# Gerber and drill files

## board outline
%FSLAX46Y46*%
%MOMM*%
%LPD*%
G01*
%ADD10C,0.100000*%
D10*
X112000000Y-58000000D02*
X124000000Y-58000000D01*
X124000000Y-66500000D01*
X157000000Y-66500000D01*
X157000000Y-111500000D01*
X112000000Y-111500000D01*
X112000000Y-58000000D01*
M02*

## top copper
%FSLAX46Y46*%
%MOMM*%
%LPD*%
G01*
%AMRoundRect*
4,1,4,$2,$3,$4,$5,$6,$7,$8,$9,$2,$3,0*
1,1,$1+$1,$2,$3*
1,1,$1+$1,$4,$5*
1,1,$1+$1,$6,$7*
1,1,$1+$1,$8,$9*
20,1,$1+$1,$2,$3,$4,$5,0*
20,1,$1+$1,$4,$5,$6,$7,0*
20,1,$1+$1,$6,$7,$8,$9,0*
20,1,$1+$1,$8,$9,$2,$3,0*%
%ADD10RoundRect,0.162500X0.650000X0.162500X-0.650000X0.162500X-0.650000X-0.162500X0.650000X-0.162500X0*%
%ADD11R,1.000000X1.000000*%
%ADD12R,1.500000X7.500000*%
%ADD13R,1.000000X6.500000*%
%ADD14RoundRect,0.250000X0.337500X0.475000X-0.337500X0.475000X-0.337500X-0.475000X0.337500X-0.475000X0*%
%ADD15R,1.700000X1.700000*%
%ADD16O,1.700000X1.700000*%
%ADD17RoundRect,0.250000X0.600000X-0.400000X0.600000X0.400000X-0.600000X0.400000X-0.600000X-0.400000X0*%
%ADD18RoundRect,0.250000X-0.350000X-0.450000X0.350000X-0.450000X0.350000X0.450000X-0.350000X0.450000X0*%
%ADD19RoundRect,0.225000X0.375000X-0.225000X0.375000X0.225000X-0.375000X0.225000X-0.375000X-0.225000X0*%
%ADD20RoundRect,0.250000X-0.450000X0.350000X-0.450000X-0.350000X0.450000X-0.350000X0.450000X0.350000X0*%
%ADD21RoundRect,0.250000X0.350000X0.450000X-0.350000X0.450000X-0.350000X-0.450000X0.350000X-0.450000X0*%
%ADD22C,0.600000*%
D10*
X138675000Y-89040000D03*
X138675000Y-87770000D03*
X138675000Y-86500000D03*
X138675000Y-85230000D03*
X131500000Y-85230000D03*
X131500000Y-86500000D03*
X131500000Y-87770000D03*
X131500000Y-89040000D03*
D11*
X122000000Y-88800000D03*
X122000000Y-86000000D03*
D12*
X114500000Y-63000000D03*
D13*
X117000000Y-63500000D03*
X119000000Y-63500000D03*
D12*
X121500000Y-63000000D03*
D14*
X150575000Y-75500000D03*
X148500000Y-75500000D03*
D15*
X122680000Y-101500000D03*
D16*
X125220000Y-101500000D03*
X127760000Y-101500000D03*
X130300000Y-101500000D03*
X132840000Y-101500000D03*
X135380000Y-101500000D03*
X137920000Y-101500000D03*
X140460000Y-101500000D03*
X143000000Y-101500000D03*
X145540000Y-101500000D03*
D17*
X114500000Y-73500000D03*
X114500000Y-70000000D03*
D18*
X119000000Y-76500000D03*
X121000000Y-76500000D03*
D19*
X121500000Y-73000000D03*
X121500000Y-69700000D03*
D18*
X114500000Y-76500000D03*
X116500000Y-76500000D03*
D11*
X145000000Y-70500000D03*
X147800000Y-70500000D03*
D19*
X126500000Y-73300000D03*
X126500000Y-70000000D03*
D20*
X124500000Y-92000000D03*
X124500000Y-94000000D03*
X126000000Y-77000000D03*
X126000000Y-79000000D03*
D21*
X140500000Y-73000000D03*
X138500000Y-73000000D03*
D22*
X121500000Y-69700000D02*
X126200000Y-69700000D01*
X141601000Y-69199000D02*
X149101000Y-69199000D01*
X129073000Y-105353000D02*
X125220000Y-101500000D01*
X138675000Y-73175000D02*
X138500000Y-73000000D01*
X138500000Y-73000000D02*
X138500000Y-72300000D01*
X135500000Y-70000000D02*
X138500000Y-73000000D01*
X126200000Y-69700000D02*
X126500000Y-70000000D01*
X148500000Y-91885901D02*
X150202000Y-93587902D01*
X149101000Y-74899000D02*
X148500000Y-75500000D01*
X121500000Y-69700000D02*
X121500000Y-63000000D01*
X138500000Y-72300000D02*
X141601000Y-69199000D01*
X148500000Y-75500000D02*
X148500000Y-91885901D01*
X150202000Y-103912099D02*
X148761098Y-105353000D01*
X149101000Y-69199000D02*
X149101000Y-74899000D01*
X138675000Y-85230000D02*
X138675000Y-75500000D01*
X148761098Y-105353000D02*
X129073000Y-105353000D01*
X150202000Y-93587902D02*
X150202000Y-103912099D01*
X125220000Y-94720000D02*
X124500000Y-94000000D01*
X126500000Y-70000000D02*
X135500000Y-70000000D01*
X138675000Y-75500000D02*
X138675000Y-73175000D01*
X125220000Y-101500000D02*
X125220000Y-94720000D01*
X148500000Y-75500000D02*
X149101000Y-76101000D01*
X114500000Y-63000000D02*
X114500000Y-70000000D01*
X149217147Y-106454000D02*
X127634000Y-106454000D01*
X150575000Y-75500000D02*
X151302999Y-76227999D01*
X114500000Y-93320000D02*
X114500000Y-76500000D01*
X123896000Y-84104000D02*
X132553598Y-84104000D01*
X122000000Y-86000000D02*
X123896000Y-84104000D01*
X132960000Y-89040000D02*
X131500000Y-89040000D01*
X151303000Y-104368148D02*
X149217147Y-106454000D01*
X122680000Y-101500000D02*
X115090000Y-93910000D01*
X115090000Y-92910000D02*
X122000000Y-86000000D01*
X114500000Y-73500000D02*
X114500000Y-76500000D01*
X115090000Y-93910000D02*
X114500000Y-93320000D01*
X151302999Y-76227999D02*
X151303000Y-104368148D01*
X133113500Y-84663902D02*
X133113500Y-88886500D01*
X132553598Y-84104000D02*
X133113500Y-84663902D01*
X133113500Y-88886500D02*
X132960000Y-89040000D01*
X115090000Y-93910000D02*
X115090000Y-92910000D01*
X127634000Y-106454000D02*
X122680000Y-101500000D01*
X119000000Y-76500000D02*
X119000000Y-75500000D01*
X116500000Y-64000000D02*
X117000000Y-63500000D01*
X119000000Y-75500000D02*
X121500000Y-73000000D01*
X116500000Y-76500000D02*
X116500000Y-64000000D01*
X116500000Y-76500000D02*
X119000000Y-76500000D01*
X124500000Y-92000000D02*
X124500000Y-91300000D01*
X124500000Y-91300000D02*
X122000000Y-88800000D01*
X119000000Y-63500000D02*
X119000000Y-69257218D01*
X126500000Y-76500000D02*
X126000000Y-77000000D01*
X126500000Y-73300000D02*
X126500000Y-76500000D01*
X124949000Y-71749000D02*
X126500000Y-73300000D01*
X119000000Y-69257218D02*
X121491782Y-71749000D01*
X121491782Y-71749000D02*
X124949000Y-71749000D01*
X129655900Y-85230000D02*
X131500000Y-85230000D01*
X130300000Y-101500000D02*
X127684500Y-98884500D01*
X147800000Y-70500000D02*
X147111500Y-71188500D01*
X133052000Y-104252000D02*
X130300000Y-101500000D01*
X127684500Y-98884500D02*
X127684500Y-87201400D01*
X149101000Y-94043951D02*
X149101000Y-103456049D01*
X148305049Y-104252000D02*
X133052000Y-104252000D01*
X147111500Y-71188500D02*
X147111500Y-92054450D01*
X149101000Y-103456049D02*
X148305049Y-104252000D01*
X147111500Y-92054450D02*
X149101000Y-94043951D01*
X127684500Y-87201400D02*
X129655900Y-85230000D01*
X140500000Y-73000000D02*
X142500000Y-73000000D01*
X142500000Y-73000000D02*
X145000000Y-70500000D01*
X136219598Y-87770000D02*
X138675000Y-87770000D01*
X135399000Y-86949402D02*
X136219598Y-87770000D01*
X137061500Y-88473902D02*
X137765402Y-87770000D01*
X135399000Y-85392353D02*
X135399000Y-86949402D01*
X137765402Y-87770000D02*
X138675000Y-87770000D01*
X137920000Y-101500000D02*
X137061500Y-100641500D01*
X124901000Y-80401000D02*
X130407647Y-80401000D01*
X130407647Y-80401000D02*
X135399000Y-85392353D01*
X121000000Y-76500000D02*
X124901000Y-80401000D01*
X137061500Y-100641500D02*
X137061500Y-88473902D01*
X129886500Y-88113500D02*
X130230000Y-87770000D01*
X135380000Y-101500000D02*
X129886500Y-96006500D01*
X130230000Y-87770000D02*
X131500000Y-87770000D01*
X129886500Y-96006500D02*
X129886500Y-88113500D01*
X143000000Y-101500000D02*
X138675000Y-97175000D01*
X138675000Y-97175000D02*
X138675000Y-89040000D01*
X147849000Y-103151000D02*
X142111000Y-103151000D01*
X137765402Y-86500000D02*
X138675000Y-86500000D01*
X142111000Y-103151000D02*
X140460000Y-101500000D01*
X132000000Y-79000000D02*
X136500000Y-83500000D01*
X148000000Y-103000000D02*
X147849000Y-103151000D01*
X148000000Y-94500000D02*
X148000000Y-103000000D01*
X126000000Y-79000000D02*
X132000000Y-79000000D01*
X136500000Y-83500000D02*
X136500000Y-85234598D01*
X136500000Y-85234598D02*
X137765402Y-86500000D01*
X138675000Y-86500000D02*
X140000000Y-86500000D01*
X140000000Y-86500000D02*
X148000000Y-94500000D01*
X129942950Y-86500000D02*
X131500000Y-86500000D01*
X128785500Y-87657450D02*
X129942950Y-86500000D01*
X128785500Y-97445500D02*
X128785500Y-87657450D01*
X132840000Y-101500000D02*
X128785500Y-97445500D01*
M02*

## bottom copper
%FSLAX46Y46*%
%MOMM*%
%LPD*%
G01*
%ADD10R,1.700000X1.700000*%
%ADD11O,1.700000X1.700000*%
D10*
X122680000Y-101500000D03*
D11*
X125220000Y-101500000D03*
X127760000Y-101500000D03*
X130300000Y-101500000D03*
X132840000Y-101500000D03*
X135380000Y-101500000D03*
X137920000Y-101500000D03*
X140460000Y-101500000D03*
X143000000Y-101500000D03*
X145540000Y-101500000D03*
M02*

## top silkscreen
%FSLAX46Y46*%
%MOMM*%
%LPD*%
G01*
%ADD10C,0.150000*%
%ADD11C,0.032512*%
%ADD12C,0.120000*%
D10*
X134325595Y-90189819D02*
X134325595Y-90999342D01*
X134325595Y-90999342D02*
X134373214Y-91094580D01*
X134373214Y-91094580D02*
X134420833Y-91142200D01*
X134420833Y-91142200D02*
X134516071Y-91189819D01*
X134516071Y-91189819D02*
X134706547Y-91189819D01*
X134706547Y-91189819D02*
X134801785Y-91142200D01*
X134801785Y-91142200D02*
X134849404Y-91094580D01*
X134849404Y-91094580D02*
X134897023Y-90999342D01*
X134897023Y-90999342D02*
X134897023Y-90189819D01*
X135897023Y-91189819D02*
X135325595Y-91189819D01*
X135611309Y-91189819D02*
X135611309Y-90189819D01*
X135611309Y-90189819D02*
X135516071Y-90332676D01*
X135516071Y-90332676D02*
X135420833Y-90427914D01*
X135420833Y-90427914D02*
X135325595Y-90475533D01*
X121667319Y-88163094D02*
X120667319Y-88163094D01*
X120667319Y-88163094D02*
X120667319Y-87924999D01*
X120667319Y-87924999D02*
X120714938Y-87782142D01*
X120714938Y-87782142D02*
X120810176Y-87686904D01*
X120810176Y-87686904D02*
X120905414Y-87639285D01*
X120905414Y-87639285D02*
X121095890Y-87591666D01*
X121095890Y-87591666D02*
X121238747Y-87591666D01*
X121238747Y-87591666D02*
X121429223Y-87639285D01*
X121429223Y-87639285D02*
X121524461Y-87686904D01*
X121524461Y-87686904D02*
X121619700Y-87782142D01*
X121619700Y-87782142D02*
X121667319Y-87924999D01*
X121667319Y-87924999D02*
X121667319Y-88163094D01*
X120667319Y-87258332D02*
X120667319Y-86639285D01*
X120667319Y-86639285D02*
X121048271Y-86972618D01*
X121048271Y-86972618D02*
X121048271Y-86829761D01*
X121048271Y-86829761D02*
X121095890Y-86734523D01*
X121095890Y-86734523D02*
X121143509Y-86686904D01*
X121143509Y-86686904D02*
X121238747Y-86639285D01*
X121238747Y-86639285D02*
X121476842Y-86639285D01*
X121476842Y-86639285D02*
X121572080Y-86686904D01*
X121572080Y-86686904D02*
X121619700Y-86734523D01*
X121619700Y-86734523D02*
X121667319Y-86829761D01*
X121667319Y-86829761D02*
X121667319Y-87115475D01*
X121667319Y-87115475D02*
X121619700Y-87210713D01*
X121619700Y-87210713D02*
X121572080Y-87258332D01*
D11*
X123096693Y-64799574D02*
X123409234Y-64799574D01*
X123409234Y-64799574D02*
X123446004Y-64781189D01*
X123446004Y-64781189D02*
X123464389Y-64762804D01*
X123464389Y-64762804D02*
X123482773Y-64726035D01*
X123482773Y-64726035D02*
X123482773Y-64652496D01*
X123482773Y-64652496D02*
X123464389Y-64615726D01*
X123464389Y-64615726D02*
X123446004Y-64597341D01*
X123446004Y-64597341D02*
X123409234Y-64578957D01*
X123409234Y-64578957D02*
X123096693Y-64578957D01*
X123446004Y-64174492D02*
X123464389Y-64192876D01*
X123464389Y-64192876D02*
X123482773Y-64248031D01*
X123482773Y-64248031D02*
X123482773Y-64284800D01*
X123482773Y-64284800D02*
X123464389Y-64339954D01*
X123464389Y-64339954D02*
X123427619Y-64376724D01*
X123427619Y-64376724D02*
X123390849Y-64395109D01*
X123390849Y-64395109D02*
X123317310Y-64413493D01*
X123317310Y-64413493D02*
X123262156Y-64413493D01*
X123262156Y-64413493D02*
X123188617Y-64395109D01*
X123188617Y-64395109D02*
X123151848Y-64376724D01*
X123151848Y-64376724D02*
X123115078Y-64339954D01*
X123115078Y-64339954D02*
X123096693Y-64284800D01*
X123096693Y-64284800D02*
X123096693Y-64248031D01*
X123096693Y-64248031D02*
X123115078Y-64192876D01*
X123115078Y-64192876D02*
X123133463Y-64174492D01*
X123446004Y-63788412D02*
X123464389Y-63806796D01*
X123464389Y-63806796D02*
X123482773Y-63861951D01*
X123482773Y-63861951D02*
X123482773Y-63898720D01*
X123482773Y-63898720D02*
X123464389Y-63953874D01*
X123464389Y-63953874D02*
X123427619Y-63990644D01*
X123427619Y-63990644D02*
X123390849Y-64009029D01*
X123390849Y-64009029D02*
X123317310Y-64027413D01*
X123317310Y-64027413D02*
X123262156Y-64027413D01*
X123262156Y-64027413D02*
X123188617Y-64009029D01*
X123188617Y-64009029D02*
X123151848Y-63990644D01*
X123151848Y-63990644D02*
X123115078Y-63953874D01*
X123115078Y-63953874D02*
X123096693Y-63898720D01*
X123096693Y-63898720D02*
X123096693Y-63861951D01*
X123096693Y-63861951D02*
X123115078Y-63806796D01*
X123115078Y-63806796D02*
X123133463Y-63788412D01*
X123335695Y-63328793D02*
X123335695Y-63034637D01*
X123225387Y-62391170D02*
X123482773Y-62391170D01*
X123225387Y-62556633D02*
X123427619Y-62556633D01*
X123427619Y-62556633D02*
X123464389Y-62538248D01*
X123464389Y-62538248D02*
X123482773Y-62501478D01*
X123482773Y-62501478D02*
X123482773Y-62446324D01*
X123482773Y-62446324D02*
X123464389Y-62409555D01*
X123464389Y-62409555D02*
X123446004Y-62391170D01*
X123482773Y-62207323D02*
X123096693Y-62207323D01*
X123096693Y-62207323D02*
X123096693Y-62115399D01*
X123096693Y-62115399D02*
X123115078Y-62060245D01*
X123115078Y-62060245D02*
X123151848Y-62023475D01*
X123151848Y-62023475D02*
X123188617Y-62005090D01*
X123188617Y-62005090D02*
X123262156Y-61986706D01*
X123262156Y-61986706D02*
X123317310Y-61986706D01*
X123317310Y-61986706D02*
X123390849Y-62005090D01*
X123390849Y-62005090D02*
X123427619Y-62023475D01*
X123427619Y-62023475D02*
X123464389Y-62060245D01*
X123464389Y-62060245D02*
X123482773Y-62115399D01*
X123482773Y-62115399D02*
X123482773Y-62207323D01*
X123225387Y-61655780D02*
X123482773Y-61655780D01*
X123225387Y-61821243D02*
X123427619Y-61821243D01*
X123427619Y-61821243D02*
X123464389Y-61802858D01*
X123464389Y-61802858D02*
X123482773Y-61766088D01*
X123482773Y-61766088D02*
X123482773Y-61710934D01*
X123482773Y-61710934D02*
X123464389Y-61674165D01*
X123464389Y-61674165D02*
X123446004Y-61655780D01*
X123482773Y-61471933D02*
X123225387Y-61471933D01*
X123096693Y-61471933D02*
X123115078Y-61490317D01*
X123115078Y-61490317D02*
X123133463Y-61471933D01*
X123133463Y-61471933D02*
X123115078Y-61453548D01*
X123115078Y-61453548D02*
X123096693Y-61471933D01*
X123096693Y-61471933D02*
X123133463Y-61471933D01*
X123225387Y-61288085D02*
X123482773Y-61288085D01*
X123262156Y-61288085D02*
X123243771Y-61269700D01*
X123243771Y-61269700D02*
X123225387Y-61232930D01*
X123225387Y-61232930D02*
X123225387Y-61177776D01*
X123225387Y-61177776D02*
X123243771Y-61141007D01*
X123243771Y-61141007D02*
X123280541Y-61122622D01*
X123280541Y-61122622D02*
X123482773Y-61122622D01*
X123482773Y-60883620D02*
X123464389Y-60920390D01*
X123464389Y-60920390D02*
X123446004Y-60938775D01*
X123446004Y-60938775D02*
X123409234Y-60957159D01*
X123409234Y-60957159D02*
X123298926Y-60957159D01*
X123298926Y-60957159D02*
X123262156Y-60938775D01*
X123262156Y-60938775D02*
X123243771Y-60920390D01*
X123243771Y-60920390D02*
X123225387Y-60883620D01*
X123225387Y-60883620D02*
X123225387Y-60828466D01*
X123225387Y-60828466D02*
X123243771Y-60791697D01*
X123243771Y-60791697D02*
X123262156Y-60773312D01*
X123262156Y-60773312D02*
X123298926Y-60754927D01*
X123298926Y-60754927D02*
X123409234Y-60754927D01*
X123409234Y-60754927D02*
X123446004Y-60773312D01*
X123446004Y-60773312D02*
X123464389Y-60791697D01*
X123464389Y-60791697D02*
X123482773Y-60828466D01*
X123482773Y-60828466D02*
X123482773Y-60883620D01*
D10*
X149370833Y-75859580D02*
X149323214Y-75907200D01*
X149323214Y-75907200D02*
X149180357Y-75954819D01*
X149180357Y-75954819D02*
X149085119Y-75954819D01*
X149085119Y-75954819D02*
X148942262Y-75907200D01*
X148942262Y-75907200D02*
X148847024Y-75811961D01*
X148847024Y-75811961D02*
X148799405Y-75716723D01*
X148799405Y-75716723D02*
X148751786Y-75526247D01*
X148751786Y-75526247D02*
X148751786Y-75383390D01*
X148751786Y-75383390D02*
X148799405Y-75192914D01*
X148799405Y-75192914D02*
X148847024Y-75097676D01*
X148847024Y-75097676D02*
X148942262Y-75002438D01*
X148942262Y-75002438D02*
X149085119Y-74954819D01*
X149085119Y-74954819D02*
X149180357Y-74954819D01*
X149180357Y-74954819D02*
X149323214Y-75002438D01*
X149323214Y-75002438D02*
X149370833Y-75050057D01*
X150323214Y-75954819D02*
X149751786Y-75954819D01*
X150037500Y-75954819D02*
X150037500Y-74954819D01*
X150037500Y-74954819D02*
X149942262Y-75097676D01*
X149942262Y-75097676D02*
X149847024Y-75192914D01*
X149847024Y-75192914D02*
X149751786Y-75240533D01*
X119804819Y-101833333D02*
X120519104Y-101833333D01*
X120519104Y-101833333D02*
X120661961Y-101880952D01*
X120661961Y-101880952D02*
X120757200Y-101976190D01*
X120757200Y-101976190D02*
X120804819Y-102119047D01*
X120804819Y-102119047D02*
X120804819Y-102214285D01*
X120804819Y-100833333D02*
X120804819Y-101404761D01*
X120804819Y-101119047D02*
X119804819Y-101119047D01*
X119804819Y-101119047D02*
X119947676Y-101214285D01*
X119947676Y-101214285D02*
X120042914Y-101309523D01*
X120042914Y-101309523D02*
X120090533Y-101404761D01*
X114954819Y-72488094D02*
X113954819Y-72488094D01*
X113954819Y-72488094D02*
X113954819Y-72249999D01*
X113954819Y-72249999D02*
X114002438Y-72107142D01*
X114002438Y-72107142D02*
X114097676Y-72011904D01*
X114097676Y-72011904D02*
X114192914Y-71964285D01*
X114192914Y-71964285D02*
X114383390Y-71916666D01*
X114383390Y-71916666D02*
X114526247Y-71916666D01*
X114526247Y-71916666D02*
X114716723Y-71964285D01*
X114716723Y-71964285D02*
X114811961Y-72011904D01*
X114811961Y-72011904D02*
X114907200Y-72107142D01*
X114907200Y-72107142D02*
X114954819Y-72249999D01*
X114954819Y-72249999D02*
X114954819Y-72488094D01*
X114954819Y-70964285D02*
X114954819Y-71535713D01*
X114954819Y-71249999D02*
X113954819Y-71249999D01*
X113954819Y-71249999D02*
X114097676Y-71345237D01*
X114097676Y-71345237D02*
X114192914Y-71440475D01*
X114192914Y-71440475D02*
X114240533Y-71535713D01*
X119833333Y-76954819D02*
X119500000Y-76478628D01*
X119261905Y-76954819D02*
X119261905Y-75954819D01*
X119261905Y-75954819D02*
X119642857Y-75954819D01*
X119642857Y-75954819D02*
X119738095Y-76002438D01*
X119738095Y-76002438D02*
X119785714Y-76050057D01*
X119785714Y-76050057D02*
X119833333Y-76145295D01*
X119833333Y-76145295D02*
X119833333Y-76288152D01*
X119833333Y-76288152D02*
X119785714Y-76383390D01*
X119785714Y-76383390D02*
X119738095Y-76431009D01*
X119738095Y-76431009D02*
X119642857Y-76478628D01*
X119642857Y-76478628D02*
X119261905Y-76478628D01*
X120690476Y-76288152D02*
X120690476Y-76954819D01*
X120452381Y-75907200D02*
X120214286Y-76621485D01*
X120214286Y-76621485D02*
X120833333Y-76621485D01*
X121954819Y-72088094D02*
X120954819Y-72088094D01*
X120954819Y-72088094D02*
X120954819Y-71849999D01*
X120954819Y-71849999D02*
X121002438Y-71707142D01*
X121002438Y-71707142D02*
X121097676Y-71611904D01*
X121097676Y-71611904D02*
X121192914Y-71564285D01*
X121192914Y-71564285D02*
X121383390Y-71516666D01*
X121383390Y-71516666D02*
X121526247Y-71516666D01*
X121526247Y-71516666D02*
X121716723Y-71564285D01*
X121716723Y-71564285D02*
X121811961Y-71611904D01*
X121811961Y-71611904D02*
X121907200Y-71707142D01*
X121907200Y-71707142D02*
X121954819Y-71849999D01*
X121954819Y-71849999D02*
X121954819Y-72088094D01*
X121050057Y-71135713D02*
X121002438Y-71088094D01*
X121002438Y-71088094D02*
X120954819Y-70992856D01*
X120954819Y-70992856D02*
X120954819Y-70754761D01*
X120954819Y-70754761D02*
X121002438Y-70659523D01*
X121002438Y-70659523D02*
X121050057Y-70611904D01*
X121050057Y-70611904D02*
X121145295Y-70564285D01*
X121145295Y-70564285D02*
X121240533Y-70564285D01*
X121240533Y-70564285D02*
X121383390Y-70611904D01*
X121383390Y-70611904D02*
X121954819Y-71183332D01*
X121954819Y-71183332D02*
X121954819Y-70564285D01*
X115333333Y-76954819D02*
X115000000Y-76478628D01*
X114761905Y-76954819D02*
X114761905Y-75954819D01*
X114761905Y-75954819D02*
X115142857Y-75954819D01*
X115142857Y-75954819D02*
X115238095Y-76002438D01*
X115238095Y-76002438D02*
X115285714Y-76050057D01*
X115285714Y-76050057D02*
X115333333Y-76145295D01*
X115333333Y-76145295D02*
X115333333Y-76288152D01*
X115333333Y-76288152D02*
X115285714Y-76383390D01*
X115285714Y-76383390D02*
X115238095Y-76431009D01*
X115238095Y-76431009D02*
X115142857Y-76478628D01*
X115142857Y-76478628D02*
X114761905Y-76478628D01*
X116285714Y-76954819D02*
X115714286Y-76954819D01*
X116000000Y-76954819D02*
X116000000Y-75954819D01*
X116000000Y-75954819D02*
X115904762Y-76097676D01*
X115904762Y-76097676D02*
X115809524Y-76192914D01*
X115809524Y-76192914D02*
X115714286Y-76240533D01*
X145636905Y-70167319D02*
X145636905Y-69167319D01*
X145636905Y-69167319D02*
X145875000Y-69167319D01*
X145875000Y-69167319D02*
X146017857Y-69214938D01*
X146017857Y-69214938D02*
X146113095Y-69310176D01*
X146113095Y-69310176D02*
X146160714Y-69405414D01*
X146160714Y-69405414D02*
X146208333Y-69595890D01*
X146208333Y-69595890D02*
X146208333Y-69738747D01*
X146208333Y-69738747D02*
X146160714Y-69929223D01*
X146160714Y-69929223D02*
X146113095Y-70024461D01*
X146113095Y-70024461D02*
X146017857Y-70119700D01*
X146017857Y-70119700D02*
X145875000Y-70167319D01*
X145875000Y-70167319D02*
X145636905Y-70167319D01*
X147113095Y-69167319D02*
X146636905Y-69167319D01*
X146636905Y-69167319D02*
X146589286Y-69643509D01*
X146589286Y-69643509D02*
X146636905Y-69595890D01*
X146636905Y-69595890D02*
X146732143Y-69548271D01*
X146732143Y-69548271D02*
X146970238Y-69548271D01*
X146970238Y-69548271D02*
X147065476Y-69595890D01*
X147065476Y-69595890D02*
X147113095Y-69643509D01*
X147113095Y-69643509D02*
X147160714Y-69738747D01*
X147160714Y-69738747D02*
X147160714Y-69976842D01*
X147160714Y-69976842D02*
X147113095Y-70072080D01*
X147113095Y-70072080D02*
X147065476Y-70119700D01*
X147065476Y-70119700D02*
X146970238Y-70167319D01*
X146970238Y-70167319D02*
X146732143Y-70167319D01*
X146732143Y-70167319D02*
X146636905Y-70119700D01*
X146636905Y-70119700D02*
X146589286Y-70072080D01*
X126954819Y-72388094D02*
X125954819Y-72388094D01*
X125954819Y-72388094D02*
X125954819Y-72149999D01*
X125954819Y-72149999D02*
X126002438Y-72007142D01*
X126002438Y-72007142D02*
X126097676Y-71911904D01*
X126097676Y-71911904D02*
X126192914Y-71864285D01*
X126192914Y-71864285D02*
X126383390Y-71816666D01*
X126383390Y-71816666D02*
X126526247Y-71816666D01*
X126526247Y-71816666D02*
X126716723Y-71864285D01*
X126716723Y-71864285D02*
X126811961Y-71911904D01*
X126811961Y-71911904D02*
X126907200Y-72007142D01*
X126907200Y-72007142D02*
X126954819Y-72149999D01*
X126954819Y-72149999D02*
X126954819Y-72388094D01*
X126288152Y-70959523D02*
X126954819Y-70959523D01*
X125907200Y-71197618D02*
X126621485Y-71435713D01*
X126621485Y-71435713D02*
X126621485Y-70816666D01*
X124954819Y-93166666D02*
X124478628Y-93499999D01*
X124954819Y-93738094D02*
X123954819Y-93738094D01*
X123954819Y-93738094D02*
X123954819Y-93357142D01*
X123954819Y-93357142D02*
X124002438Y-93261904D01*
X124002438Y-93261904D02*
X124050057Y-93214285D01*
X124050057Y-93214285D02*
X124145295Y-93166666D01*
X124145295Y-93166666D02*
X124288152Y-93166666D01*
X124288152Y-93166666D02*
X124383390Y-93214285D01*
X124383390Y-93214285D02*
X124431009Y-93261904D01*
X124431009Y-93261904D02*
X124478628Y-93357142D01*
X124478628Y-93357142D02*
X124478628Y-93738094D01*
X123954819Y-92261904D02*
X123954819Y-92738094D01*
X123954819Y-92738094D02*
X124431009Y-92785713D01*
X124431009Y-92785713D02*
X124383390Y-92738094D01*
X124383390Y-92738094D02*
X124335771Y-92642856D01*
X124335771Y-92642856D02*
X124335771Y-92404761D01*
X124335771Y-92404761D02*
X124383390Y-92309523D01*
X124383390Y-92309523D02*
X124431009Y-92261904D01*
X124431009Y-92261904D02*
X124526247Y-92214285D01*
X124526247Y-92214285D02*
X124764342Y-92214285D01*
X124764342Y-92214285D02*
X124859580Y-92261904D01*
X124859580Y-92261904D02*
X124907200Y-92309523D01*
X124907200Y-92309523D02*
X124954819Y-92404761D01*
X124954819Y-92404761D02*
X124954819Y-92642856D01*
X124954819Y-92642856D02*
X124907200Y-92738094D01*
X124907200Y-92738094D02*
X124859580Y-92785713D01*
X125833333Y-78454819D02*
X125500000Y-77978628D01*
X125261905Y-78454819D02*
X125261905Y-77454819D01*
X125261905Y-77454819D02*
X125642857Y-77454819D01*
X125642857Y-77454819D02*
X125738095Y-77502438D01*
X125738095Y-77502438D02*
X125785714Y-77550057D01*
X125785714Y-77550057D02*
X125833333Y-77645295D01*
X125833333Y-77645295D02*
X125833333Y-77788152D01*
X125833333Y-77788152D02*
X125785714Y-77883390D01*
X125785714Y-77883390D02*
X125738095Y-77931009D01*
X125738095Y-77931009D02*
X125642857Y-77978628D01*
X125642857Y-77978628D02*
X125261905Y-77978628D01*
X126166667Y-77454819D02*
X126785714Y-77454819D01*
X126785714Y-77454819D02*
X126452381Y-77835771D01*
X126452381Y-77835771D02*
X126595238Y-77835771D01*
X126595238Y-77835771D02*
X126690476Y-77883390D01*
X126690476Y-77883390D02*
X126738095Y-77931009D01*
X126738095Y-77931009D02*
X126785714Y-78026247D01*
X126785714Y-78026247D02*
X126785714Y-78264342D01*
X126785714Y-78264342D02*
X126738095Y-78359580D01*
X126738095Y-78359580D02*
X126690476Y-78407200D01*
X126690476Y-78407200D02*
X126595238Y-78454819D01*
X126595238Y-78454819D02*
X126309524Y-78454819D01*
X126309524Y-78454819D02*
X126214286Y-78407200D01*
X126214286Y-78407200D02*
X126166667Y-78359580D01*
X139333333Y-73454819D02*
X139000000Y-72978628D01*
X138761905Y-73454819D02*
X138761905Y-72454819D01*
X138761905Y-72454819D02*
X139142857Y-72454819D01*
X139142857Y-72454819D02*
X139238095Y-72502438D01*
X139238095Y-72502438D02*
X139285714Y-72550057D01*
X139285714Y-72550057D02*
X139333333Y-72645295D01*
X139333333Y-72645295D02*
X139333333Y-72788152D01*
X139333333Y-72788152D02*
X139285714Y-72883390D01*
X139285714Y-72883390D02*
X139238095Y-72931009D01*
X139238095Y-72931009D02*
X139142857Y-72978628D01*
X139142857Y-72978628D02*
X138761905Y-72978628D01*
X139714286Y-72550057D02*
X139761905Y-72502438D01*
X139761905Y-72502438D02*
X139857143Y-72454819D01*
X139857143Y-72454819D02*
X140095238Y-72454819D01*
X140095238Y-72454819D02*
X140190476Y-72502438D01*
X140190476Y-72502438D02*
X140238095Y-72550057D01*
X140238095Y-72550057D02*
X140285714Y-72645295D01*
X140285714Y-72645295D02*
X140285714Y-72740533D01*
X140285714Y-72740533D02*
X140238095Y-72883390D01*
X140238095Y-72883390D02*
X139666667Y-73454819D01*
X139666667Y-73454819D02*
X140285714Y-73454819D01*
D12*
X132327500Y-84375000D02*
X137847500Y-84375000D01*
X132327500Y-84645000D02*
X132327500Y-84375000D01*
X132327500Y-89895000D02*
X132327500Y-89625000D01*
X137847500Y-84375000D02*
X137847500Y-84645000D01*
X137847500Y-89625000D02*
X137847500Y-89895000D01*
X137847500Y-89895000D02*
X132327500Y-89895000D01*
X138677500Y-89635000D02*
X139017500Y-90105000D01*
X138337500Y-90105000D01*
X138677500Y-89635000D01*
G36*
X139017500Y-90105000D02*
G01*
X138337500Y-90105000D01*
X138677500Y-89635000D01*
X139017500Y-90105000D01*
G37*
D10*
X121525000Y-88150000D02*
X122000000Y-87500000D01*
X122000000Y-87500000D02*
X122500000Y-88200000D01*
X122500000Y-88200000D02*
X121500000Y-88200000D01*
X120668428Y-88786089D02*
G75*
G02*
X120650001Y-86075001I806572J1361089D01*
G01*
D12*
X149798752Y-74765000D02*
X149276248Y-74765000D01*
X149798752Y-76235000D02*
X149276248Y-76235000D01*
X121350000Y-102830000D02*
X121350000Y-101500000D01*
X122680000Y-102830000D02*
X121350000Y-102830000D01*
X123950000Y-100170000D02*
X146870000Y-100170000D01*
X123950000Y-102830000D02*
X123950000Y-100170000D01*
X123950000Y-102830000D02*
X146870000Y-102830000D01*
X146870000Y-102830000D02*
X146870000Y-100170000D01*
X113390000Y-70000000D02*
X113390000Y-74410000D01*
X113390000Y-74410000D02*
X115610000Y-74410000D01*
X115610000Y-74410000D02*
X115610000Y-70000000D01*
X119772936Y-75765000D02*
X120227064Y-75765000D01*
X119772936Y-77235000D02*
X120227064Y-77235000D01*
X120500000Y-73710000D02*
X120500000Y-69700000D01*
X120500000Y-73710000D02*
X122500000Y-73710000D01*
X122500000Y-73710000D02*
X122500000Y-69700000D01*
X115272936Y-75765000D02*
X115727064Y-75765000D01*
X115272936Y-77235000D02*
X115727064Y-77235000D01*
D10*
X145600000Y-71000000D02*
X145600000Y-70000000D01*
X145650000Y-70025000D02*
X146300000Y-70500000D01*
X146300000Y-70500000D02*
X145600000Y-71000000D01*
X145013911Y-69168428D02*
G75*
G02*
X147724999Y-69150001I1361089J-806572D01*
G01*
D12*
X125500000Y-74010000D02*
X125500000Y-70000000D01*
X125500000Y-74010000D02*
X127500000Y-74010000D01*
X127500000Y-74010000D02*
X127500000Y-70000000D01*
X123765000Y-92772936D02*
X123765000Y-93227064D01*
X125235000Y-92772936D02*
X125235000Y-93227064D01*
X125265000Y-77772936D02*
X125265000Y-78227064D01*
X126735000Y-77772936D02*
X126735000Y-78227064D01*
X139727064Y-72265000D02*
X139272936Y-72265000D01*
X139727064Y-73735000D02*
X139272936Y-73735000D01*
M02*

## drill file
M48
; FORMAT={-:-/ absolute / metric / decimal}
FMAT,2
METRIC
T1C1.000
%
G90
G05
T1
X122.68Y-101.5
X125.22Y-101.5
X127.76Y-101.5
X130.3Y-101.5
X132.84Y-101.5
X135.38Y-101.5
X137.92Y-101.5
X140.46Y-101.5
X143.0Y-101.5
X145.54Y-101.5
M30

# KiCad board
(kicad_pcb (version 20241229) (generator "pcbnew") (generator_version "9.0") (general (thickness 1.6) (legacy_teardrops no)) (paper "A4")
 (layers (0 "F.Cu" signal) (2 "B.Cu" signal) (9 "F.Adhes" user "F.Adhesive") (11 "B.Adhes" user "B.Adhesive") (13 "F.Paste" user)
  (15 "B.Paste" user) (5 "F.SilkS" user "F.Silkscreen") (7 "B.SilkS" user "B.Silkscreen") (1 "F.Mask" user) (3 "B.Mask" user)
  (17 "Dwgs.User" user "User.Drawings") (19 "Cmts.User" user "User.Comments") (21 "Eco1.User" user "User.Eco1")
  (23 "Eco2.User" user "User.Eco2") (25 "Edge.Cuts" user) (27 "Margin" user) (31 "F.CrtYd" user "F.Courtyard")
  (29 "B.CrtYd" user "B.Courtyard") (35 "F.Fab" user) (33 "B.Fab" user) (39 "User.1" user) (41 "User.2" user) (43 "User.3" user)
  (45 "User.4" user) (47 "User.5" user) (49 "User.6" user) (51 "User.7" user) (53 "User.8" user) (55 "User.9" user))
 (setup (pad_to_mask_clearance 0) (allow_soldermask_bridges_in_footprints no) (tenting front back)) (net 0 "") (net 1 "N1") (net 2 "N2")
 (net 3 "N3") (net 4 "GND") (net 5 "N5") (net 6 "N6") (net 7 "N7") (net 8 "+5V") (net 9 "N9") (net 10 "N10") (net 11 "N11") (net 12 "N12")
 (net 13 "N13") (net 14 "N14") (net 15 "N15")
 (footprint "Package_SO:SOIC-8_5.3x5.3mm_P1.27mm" (layer "F.Cu") (at 135.0875 87.135 180)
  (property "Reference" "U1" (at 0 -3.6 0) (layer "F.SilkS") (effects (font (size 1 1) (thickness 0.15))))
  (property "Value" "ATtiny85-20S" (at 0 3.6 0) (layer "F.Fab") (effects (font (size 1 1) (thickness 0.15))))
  (fp_line (start 2.76 2.76) (end -2.76 2.76) (stroke (width 0.12) (type solid)) (layer "F.SilkS"))
  (fp_line (start 2.76 2.49) (end 2.76 2.76) (stroke (width 0.12) (type solid)) (layer "F.SilkS"))
  (fp_line (start 2.76 -2.76) (end 2.76 -2.49) (stroke (width 0.12) (type solid)) (layer "F.SilkS"))
  (fp_line (start -2.76 2.76) (end -2.76 2.49) (stroke (width 0.12) (type solid)) (layer "F.SilkS"))
  (fp_line (start -2.76 -2.49) (end -2.76 -2.76) (stroke (width 0.12) (type solid)) (layer "F.SilkS"))
  (fp_line (start -2.76 -2.76) (end 2.76 -2.76) (stroke (width 0.12) (type solid)) (layer "F.SilkS"))
  (fp_poly (pts (xy -3.59 -2.5) (xy -3.93 -2.97) (xy -3.25 -2.97)) (stroke (width 0.12) (type solid)) (fill yes) (layer "F.SilkS"))
  (pad "1" smd roundrect (at -3.5875 -1.905 180) (size 1.625 0.65) (layers "F.Cu" "F.Mask" "F.Paste") (roundrect_rratio 0.25) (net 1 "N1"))
  (pad "2" smd roundrect (at -3.5875 -0.635 180) (size 1.625 0.65) (layers "F.Cu" "F.Mask" "F.Paste") (roundrect_rratio 0.25) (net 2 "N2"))
  (pad "3" smd roundrect (at -3.5875 0.635 180) (size 1.625 0.65) (layers "F.Cu" "F.Mask" "F.Paste") (roundrect_rratio 0.25) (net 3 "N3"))
  (pad "4" smd roundrect (at -3.5875 1.905 180) (size 1.625 0.65) (layers "F.Cu" "F.Mask" "F.Paste") (roundrect_rratio 0.25) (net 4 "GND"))
  (pad "5" smd roundrect (at 3.5875 1.905 180) (size 1.625 0.65) (layers "F.Cu" "F.Mask" "F.Paste") (roundrect_rratio 0.25) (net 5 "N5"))
  (pad "6" smd roundrect (at 3.5875 0.635 180) (size 1.625 0.65) (layers "F.Cu" "F.Mask" "F.Paste") (roundrect_rratio 0.25) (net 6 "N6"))
  (pad "7" smd roundrect (at 3.5875 -0.635 180) (size 1.625 0.65) (layers "F.Cu" "F.Mask" "F.Paste") (roundrect_rratio 0.25) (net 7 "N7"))
  (pad "8" smd roundrect (at 3.5875 -1.905 180) (size 1.625 0.65) (layers "F.Cu" "F.Mask" "F.Paste") (roundrect_rratio 0.25) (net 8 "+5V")))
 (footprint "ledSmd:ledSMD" (layer "F.Cu") (at 122 87 90)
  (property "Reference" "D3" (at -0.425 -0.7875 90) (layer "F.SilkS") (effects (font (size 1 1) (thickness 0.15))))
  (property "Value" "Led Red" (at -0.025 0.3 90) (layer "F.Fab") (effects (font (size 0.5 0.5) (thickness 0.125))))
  (fp_line (start -1.15 -0.475) (end -0.5 0) (stroke (width 0.15) (type solid)) (layer "F.SilkS"))
  (fp_line (start -0.5 0) (end -1.2 0.5) (stroke (width 0.15) (type solid)) (layer "F.SilkS"))
  (fp_line (start -1.2 0.5) (end -1.2 -0.5) (stroke (width 0.15) (type solid)) (layer "F.SilkS"))
  (fp_arc (start -1.786089 -1.331572) (mid -0.435753 -2.107089) (end 0.924999 -1.349999) (stroke (width 0.15) (type solid))
   (layer "F.SilkS"))
  (pad "1" smd rect (at -1.8 0 90) (size 1 1) (layers "F.Cu" "F.Mask" "F.Paste") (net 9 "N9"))
  (pad "2" smd rect (at 1 0 90) (size 1 1) (layers "F.Cu" "F.Mask" "F.Paste") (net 8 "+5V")))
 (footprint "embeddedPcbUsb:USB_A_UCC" (layer "F.Cu") (at 118 63.2 -90)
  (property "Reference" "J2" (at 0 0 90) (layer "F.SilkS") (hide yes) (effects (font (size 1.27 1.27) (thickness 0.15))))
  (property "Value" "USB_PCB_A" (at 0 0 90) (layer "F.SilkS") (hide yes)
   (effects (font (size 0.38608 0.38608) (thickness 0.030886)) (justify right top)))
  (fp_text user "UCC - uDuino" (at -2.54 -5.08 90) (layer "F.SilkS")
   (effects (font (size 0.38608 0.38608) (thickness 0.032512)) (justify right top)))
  (pad "1" smd rect (at -0.2 3.5 270) (size 7.5 1.5) (layers "F.Cu" "F.Mask" "F.Paste") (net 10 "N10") (solder_mask_margin 0.1016))
  (pad "2" smd rect (at 0.3 1 270) (size 6.5 1) (layers "F.Cu" "F.Mask" "F.Paste") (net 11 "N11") (solder_mask_margin 0.1016))
  (pad "3" smd rect (at 0.3 -1 270) (size 6.5 1) (layers "F.Cu" "F.Mask" "F.Paste") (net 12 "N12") (solder_mask_margin 0.1016))
  (pad "4" smd rect (at -0.2 -3.5 270) (size 7.5 1.5) (layers "F.Cu" "F.Mask" "F.Paste") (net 4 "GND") (solder_mask_margin 0.1016)))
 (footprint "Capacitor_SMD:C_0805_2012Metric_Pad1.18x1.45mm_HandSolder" (layer "F.Cu") (at 149.5375 75.5 180)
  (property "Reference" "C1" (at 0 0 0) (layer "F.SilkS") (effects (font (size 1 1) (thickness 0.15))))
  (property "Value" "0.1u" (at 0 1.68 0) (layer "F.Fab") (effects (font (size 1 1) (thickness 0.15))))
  (fp_line (start -0.261252 0.735) (end 0.261252 0.735) (stroke (width 0.12) (type solid)) (layer "F.SilkS"))
  (fp_line (start -0.261252 -0.735) (end 0.261252 -0.735) (stroke (width 0.12) (type solid)) (layer "F.SilkS"))
  (pad "1" smd roundrect (at -1.0375 0 180) (size 1.175 1.45) (layers "F.Cu" "F.Mask" "F.Paste") (roundrect_rratio 0.212766) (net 8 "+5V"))
  (pad "2" smd roundrect (at 1.0375 0 180) (size 1.175 1.45) (layers "F.Cu" "F.Mask" "F.Paste") (roundrect_rratio 0.212766) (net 4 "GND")))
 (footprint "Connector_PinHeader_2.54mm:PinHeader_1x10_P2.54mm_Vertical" (layer "F.Cu") (at 122.68 101.5 90)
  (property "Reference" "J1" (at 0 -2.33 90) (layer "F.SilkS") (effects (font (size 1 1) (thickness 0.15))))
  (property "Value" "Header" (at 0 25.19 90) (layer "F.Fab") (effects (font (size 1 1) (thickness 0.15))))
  (fp_line (start -1.33 -1.33) (end 0 -1.33) (stroke (width 0.12) (type solid)) (layer "F.SilkS"))
  (fp_line (start -1.33 0) (end -1.33 -1.33) (stroke (width 0.12) (type solid)) (layer "F.SilkS"))
  (fp_line (start 1.33 1.27) (end 1.33 24.19) (stroke (width 0.12) (type solid)) (layer "F.SilkS"))
  (fp_line (start -1.33 1.27) (end 1.33 1.27) (stroke (width 0.12) (type solid)) (layer "F.SilkS"))
  (fp_line (start -1.33 1.27) (end -1.33 24.19) (stroke (width 0.12) (type solid)) (layer "F.SilkS"))
  (fp_line (start -1.33 24.19) (end 1.33 24.19) (stroke (width 0.12) (type solid)) (layer "F.SilkS"))
  (pad "1" thru_hole rect (at 0 0 90) (size 1.7 1.7) (drill 1) (layers "*.Cu" "*.Mask") (remove_unused_layers no) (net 8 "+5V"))
  (pad "2" thru_hole oval (at 0 2.54 90) (size 1.7 1.7) (drill 1) (layers "*.Cu" "*.Mask") (remove_unused_layers no) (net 4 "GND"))
  (pad "3" thru_hole oval (at 0 5.08 90) (size 1.7 1.7) (drill 1) (layers "*.Cu" "*.Mask") (remove_unused_layers no) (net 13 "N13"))
  (pad "4" thru_hole oval (at 0 7.62 90) (size 1.7 1.7) (drill 1) (layers "*.Cu" "*.Mask") (remove_unused_layers no) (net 5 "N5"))
  (pad "5" thru_hole oval (at 0 10.16 90) (size 1.7 1.7) (drill 1) (layers "*.Cu" "*.Mask") (remove_unused_layers no) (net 6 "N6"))
  (pad "6" thru_hole oval (at 0 12.7 90) (size 1.7 1.7) (drill 1) (layers "*.Cu" "*.Mask") (remove_unused_layers no) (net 7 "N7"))
  (pad "7" thru_hole oval (at 0 15.24 90) (size 1.7 1.7) (drill 1) (layers "*.Cu" "*.Mask") (remove_unused_layers no) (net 2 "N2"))
  (pad "8" thru_hole oval (at 0 17.78 90) (size 1.7 1.7) (drill 1) (layers "*.Cu" "*.Mask") (remove_unused_layers no) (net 3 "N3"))
  (pad "9" thru_hole oval (at 0 20.32 90) (size 1.7 1.7) (drill 1) (layers "*.Cu" "*.Mask") (remove_unused_layers no) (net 1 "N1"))
  (pad "10" thru_hole oval (at 0 22.86 90) (size 1.7 1.7) (drill 1) (layers "*.Cu" "*.Mask") (remove_unused_layers no) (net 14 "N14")))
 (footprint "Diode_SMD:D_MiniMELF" (layer "F.Cu") (at 114.5 71.75 90)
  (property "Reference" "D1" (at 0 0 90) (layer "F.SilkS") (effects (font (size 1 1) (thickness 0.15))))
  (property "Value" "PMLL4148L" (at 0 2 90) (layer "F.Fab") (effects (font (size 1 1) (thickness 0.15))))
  (fp_line (start 1.75 -1.11) (end -2.66 -1.11) (stroke (width 0.12) (type solid)) (layer "F.SilkS"))
  (fp_line (start -2.66 -1.11) (end -2.66 1.11) (stroke (width 0.12) (type solid)) (layer "F.SilkS"))
  (fp_line (start -2.66 1.11) (end 1.75 1.11) (stroke (width 0.12) (type solid)) (layer "F.SilkS"))
  (pad "1" smd roundrect (at -1.75 0 90) (size 1.3 1.7) (layers "F.Cu" "F.Mask" "F.Paste") (roundrect_rratio 0.1923076923) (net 8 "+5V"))
  (pad "2" smd roundrect (at 1.75 0 90) (size 1.3 1.7) (layers "F.Cu" "F.Mask" "F.Paste") (roundrect_rratio 0.1923076923) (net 10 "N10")))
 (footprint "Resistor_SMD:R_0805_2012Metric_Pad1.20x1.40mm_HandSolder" (layer "F.Cu") (at 120 76.5)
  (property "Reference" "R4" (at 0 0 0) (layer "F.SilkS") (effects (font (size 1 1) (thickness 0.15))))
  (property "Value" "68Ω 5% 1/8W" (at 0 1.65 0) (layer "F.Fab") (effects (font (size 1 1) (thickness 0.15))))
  (fp_line (start -0.227064 -0.735) (end 0.227064 -0.735) (stroke (width 0.12) (type solid)) (layer "F.SilkS"))
  (fp_line (start -0.227064 0.735) (end 0.227064 0.735) (stroke (width 0.12) (type solid)) (layer "F.SilkS"))
  (pad "1" smd roundrect (at -1 0) (size 1.2 1.4) (layers "F.Cu" "F.Mask" "F.Paste") (roundrect_rratio 0.208333) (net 11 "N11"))
  (pad "2" smd roundrect (at 1 0) (size 1.2 1.4) (layers "F.Cu" "F.Mask" "F.Paste") (roundrect_rratio 0.208333) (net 2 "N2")))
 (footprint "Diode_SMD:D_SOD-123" (layer "F.Cu") (at 121.5 71.35 90)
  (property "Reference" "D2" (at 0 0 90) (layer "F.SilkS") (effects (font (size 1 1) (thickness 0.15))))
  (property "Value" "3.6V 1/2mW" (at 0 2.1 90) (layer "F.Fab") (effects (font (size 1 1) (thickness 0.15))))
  (fp_line (start -2.36 -1) (end 1.65 -1) (stroke (width 0.12) (type solid)) (layer "F.SilkS"))
  (fp_line (start -2.36 -1) (end -2.36 1) (stroke (width 0.12) (type solid)) (layer "F.SilkS"))
  (fp_line (start -2.36 1) (end 1.65 1) (stroke (width 0.12) (type solid)) (layer "F.SilkS"))
  (pad "1" smd roundrect (at -1.65 0 90) (size 0.9 1.2) (layers "F.Cu" "F.Mask" "F.Paste") (roundrect_rratio 0.25) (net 11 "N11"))
  (pad "2" smd roundrect (at 1.65 0 90) (size 0.9 1.2) (layers "F.Cu" "F.Mask" "F.Paste") (roundrect_rratio 0.25) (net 4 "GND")))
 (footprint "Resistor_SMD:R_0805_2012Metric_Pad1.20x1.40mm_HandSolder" (layer "F.Cu") (at 115.5 76.5)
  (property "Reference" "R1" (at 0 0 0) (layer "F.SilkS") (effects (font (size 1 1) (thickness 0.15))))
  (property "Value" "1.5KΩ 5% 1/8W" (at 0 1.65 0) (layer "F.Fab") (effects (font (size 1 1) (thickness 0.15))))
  (fp_line (start -0.227064 -0.735) (end 0.227064 -0.735) (stroke (width 0.12) (type solid)) (layer "F.SilkS"))
  (fp_line (start -0.227064 0.735) (end 0.227064 0.735) (stroke (width 0.12) (type solid)) (layer "F.SilkS"))
  (pad "1" smd roundrect (at -1 0) (size 1.2 1.4) (layers "F.Cu" "F.Mask" "F.Paste") (roundrect_rratio 0.208333) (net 8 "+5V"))
  (pad "2" smd roundrect (at 1 0) (size 1.2 1.4) (layers "F.Cu" "F.Mask" "F.Paste") (roundrect_rratio 0.208333) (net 11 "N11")))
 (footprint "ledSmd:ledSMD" (layer "F.Cu") (at 146.8 70.5)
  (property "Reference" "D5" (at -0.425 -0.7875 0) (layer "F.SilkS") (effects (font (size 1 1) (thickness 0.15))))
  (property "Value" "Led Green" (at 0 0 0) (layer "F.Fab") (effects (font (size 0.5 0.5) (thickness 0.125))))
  (fp_line (start -1.2 0.5) (end -1.2 -0.5) (stroke (width 0.15) (type solid)) (layer "F.SilkS"))
  (fp_line (start -1.15 -0.475) (end -0.5 0) (stroke (width 0.15) (type solid)) (layer "F.SilkS"))
  (fp_line (start -0.5 0) (end -1.2 0.5) (stroke (width 0.15) (type solid)) (layer "F.SilkS"))
  (fp_arc (start -1.786089 -1.331572) (mid -0.435753 -2.107089) (end 0.924999 -1.349999) (stroke (width 0.15) (type solid))
   (layer "F.SilkS"))
  (pad "1" smd rect (at -1.8 0) (size 1 1) (layers "F.Cu" "F.Mask" "F.Paste") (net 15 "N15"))
  (pad "2" smd rect (at 1 0) (size 1 1) (layers "F.Cu" "F.Mask" "F.Paste") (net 5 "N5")))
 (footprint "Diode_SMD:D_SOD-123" (layer "F.Cu") (at 126.5 71.65 90)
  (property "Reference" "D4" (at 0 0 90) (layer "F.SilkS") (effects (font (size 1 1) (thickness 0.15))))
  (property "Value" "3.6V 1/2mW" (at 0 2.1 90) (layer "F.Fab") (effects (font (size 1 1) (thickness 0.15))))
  (fp_line (start -2.36 -1) (end 1.65 -1) (stroke (width 0.12) (type solid)) (layer "F.SilkS"))
  (fp_line (start -2.36 -1) (end -2.36 1) (stroke (width 0.12) (type solid)) (layer "F.SilkS"))
  (fp_line (start -2.36 1) (end 1.65 1) (stroke (width 0.12) (type solid)) (layer "F.SilkS"))
  (pad "1" smd roundrect (at -1.65 0 90) (size 0.9 1.2) (layers "F.Cu" "F.Mask" "F.Paste") (roundrect_rratio 0.25) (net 12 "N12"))
  (pad "2" smd roundrect (at 1.65 0 90) (size 0.9 1.2) (layers "F.Cu" "F.Mask" "F.Paste") (roundrect_rratio 0.25) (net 4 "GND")))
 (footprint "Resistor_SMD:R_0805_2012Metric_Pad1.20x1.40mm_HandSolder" (layer "F.Cu") (at 124.5 93 -90)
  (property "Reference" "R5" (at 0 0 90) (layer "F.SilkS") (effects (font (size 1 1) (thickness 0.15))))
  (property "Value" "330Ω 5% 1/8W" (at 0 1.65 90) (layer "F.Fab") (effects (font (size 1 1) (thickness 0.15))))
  (fp_line (start -0.227064 0.735) (end 0.227064 0.735) (stroke (width 0.12) (type solid)) (layer "F.SilkS"))
  (fp_line (start -0.227064 -0.735) (end 0.227064 -0.735) (stroke (width 0.12) (type solid)) (layer "F.SilkS"))
  (pad "1" smd roundrect (at -1 0 270) (size 1.2 1.4) (layers "F.Cu" "F.Mask" "F.Paste") (roundrect_rratio 0.208333) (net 9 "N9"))
  (pad "2" smd roundrect (at 1 0 270) (size 1.2 1.4) (layers "F.Cu" "F.Mask" "F.Paste") (roundrect_rratio 0.208333) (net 4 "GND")))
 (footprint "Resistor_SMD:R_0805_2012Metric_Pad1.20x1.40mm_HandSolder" (layer "F.Cu") (at 126 78 -90)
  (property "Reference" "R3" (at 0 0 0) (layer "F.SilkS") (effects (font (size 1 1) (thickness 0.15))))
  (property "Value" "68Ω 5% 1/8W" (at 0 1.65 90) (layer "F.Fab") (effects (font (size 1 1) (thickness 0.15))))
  (fp_line (start -0.227064 0.735) (end 0.227064 0.735) (stroke (width 0.12) (type solid)) (layer "F.SilkS"))
  (fp_line (start -0.227064 -0.735) (end 0.227064 -0.735) (stroke (width 0.12) (type solid)) (layer "F.SilkS"))
  (pad "1" smd roundrect (at -1 0 270) (size 1.2 1.4) (layers "F.Cu" "F.Mask" "F.Paste") (roundrect_rratio 0.208333) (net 12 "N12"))
  (pad "2" smd roundrect (at 1 0 270) (size 1.2 1.4) (layers "F.Cu" "F.Mask" "F.Paste") (roundrect_rratio 0.208333) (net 3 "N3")))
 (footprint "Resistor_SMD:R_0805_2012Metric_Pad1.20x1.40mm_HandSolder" (layer "F.Cu") (at 139.5 73 180)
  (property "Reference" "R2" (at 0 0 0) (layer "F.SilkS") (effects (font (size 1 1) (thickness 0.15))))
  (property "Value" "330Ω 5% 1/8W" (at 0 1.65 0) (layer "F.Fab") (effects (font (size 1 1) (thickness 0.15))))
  (fp_line (start -0.227064 0.735) (end 0.227064 0.735) (stroke (width 0.12) (type solid)) (layer "F.SilkS"))
  (fp_line (start -0.227064 -0.735) (end 0.227064 -0.735) (stroke (width 0.12) (type solid)) (layer "F.SilkS"))
  (pad "1" smd roundrect (at -1 0 180) (size 1.2 1.4) (layers "F.Cu" "F.Mask" "F.Paste") (roundrect_rratio 0.208333) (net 15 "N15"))
  (pad "2" smd roundrect (at 1 0 180) (size 1.2 1.4) (layers "F.Cu" "F.Mask" "F.Paste") (roundrect_rratio 0.208333) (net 4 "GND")))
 (gr_poly
  (pts (xy 112 58) (xy 124 58) (xy 124 66.5) (xy 157 66.5) (xy 157 111.5) (xy 112 111.5)) (stroke (width 0.1) (type solid)) (fill no)
  (layer "Edge.Cuts"))
 (segment (start 121.5 69.7) (end 126.2 69.7) (width 0.6) (layer "F.Cu") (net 4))
 (segment (start 141.601 69.199) (end 149.101 69.199) (width 0.6) (layer "F.Cu") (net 4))
 (segment (start 129.073 105.353) (end 125.22 101.5) (width 0.6) (layer "F.Cu") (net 4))
 (segment (start 138.675 73.175) (end 138.5 73) (width 0.6) (layer "F.Cu") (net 4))
 (segment (start 138.5 73) (end 138.5 72.3) (width 0.6) (layer "F.Cu") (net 4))
 (segment (start 135.5 70) (end 138.5 73) (width 0.6) (layer "F.Cu") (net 4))
 (segment (start 126.2 69.7) (end 126.5 70) (width 0.6) (layer "F.Cu") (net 4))
 (segment (start 148.5 91.885901) (end 150.202 93.587902) (width 0.6) (layer "F.Cu") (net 4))
 (segment (start 149.101 74.899) (end 148.5 75.5) (width 0.6) (layer "F.Cu") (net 4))
 (segment (start 121.5 69.7) (end 121.5 63) (width 0.6) (layer "F.Cu") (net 4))
 (segment (start 138.5 72.3) (end 141.601 69.199) (width 0.6) (layer "F.Cu") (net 4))
 (segment (start 148.5 75.5) (end 148.5 91.885901) (width 0.6) (layer "F.Cu") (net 4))
 (segment (start 150.202 103.912099) (end 148.761098 105.353) (width 0.6) (layer "F.Cu") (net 4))
 (segment (start 149.101 69.199) (end 149.101 74.899) (width 0.6) (layer "F.Cu") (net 4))
 (segment (start 138.675 85.23) (end 138.675 75.5) (width 0.6) (layer "F.Cu") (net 4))
 (segment (start 148.761098 105.353) (end 129.073 105.353) (width 0.6) (layer "F.Cu") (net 4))
 (segment (start 150.202 93.587902) (end 150.202 103.912099) (width 0.6) (layer "F.Cu") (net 4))
 (segment (start 125.22 94.72) (end 124.5 94) (width 0.6) (layer "F.Cu") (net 4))
 (segment (start 126.5 70) (end 135.5 70) (width 0.6) (layer "F.Cu") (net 4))
 (segment (start 138.675 75.5) (end 138.675 73.175) (width 0.6) (layer "F.Cu") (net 4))
 (segment (start 125.22 101.5) (end 125.22 94.72) (width 0.6) (layer "F.Cu") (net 4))
 (segment (start 148.5 75.5) (end 149.101 76.101) (width 0.6) (layer "F.Cu") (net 4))
 (segment (start 114.5 63) (end 114.5 70) (width 0.6) (layer "F.Cu") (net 10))
 (segment (start 149.217147 106.454) (end 127.634 106.454) (width 0.6) (layer "F.Cu") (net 8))
 (segment (start 150.575 75.5) (end 151.302999 76.227999) (width 0.6) (layer "F.Cu") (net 8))
 (segment (start 114.5 93.32) (end 114.5 76.5) (width 0.6) (layer "F.Cu") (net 8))
 (segment (start 123.896 84.104) (end 132.553598 84.104) (width 0.6) (layer "F.Cu") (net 8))
 (segment (start 122 86) (end 123.896 84.104) (width 0.6) (layer "F.Cu") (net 8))
 (segment (start 132.96 89.04) (end 131.5 89.04) (width 0.6) (layer "F.Cu") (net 8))
 (segment (start 151.303 104.368148) (end 149.217147 106.454) (width 0.6) (layer "F.Cu") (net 8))
 (segment (start 122.68 101.5) (end 115.09 93.91) (width 0.6) (layer "F.Cu") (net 8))
 (segment (start 115.09 92.91) (end 122 86) (width 0.6) (layer "F.Cu") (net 8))
 (segment (start 114.5 73.5) (end 114.5 76.5) (width 0.6) (layer "F.Cu") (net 8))
 (segment (start 115.09 93.91) (end 114.5 93.32) (width 0.6) (layer "F.Cu") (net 8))
 (segment (start 151.302999 76.227999) (end 151.303 104.368148) (width 0.6) (layer "F.Cu") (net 8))
 (segment (start 133.1135 84.663902) (end 133.1135 88.8865) (width 0.6) (layer "F.Cu") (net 8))
 (segment (start 132.553598 84.104) (end 133.1135 84.663902) (width 0.6) (layer "F.Cu") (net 8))
 (segment (start 133.1135 88.8865) (end 132.96 89.04) (width 0.6) (layer "F.Cu") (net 8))
 (segment (start 115.09 93.91) (end 115.09 92.91) (width 0.6) (layer "F.Cu") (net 8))
 (segment (start 127.634 106.454) (end 122.68 101.5) (width 0.6) (layer "F.Cu") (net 8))
 (segment (start 119 76.5) (end 119 75.5) (width 0.6) (layer "F.Cu") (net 11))
 (segment (start 116.5 64) (end 117 63.5) (width 0.6) (layer "F.Cu") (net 11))
 (segment (start 119 75.5) (end 121.5 73) (width 0.6) (layer "F.Cu") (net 11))
 (segment (start 116.5 76.5) (end 116.5 64) (width 0.6) (layer "F.Cu") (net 11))
 (segment (start 116.5 76.5) (end 119 76.5) (width 0.6) (layer "F.Cu") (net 11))
 (segment (start 124.5 92) (end 124.5 91.3) (width 0.6) (layer "F.Cu") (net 9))
 (segment (start 124.5 91.3) (end 122 88.8) (width 0.6) (layer "F.Cu") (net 9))
 (segment (start 119 63.5) (end 119 69.257218) (width 0.6) (layer "F.Cu") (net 12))
 (segment (start 126.5 76.5) (end 126 77) (width 0.6) (layer "F.Cu") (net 12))
 (segment (start 126.5 73.3) (end 126.5 76.5) (width 0.6) (layer "F.Cu") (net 12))
 (segment (start 124.949 71.749) (end 126.5 73.3) (width 0.6) (layer "F.Cu") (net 12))
 (segment (start 119 69.257218) (end 121.491782 71.749) (width 0.6) (layer "F.Cu") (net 12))
 (segment (start 121.491782 71.749) (end 124.949 71.749) (width 0.6) (layer "F.Cu") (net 12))
 (segment (start 129.6559 85.23) (end 131.5 85.23) (width 0.6) (layer "F.Cu") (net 5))
 (segment (start 130.3 101.5) (end 127.6845 98.8845) (width 0.6) (layer "F.Cu") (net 5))
 (segment (start 147.8 70.5) (end 147.1115 71.1885) (width 0.6) (layer "F.Cu") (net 5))
 (segment (start 133.052 104.252) (end 130.3 101.5) (width 0.6) (layer "F.Cu") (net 5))
 (segment (start 127.6845 98.8845) (end 127.6845 87.2014) (width 0.6) (layer "F.Cu") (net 5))
 (segment (start 149.101 94.043951) (end 149.101 103.456049) (width 0.6) (layer "F.Cu") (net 5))
 (segment (start 148.305049 104.252) (end 133.052 104.252) (width 0.6) (layer "F.Cu") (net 5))
 (segment (start 147.1115 71.1885) (end 147.1115 92.05445) (width 0.6) (layer "F.Cu") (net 5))
 (segment (start 149.101 103.456049) (end 148.305049 104.252) (width 0.6) (layer "F.Cu") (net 5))
 (segment (start 147.1115 92.05445) (end 149.101 94.043951) (width 0.6) (layer "F.Cu") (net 5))
 (segment (start 127.6845 87.2014) (end 129.6559 85.23) (width 0.6) (layer "F.Cu") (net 5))
 (segment (start 140.5 73) (end 142.5 73) (width 0.6) (layer "F.Cu") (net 15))
 (segment (start 142.5 73) (end 145 70.5) (width 0.6) (layer "F.Cu") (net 15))
 (segment (start 136.219598 87.77) (end 138.675 87.77) (width 0.6) (layer "F.Cu") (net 2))
 (segment (start 135.399 86.949402) (end 136.219598 87.77) (width 0.6) (layer "F.Cu") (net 2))
 (segment (start 137.0615 88.473902) (end 137.765402 87.77) (width 0.6) (layer "F.Cu") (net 2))
 (segment (start 135.399 85.392353) (end 135.399 86.949402) (width 0.6) (layer "F.Cu") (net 2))
 (segment (start 137.765402 87.77) (end 138.675 87.77) (width 0.6) (layer "F.Cu") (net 2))
 (segment (start 137.92 101.5) (end 137.0615 100.6415) (width 0.6) (layer "F.Cu") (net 2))
 (segment (start 124.901 80.401) (end 130.407647 80.401) (width 0.6) (layer "F.Cu") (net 2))
 (segment (start 130.407647 80.401) (end 135.399 85.392353) (width 0.6) (layer "F.Cu") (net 2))
 (segment (start 121 76.5) (end 124.901 80.401) (width 0.6) (layer "F.Cu") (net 2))
 (segment (start 137.0615 100.6415) (end 137.0615 88.473902) (width 0.6) (layer "F.Cu") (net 2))
 (segment (start 129.8865 88.1135) (end 130.23 87.77) (width 0.6) (layer "F.Cu") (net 7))
 (segment (start 135.38 101.5) (end 129.8865 96.0065) (width 0.6) (layer "F.Cu") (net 7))
 (segment (start 130.23 87.77) (end 131.5 87.77) (width 0.6) (layer "F.Cu") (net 7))
 (segment (start 129.8865 96.0065) (end 129.8865 88.1135) (width 0.6) (layer "F.Cu") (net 7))
 (segment (start 143 101.5) (end 138.675 97.175) (width 0.6) (layer "F.Cu") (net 1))
 (segment (start 138.675 97.175) (end 138.675 89.04) (width 0.6) (layer "F.Cu") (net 1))
 (segment (start 147.849 103.151) (end 142.111 103.151) (width 0.6) (layer "F.Cu") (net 3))
 (segment (start 137.765402 86.5) (end 138.675 86.5) (width 0.6) (layer "F.Cu") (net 3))
 (segment (start 142.111 103.151) (end 140.46 101.5) (width 0.6) (layer "F.Cu") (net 3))
 (segment (start 132 79) (end 136.5 83.5) (width 0.6) (layer "F.Cu") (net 3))
 (segment (start 148 103) (end 147.849 103.151) (width 0.6) (layer "F.Cu") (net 3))
 (segment (start 148 94.5) (end 148 103) (width 0.6) (layer "F.Cu") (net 3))
 (segment (start 126 79) (end 132 79) (width 0.6) (layer "F.Cu") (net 3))
 (segment (start 136.5 83.5) (end 136.5 85.234598) (width 0.6) (layer "F.Cu") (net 3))
 (segment (start 136.5 85.234598) (end 137.765402 86.5) (width 0.6) (layer "F.Cu") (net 3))
 (segment (start 138.675 86.5) (end 140 86.5) (width 0.6) (layer "F.Cu") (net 3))
 (segment (start 140 86.5) (end 148 94.5) (width 0.6) (layer "F.Cu") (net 3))
 (segment (start 129.94295 86.5) (end 131.5 86.5) (width 0.6) (layer "F.Cu") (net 6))
 (segment (start 128.7855 87.65745) (end 129.94295 86.5) (width 0.6) (layer "F.Cu") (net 6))
 (segment (start 128.7855 97.4455) (end 128.7855 87.65745) (width 0.6) (layer "F.Cu") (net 6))
 (segment (start 132.84 101.5) (end 128.7855 97.4455) (width 0.6) (layer "F.Cu") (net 6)))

